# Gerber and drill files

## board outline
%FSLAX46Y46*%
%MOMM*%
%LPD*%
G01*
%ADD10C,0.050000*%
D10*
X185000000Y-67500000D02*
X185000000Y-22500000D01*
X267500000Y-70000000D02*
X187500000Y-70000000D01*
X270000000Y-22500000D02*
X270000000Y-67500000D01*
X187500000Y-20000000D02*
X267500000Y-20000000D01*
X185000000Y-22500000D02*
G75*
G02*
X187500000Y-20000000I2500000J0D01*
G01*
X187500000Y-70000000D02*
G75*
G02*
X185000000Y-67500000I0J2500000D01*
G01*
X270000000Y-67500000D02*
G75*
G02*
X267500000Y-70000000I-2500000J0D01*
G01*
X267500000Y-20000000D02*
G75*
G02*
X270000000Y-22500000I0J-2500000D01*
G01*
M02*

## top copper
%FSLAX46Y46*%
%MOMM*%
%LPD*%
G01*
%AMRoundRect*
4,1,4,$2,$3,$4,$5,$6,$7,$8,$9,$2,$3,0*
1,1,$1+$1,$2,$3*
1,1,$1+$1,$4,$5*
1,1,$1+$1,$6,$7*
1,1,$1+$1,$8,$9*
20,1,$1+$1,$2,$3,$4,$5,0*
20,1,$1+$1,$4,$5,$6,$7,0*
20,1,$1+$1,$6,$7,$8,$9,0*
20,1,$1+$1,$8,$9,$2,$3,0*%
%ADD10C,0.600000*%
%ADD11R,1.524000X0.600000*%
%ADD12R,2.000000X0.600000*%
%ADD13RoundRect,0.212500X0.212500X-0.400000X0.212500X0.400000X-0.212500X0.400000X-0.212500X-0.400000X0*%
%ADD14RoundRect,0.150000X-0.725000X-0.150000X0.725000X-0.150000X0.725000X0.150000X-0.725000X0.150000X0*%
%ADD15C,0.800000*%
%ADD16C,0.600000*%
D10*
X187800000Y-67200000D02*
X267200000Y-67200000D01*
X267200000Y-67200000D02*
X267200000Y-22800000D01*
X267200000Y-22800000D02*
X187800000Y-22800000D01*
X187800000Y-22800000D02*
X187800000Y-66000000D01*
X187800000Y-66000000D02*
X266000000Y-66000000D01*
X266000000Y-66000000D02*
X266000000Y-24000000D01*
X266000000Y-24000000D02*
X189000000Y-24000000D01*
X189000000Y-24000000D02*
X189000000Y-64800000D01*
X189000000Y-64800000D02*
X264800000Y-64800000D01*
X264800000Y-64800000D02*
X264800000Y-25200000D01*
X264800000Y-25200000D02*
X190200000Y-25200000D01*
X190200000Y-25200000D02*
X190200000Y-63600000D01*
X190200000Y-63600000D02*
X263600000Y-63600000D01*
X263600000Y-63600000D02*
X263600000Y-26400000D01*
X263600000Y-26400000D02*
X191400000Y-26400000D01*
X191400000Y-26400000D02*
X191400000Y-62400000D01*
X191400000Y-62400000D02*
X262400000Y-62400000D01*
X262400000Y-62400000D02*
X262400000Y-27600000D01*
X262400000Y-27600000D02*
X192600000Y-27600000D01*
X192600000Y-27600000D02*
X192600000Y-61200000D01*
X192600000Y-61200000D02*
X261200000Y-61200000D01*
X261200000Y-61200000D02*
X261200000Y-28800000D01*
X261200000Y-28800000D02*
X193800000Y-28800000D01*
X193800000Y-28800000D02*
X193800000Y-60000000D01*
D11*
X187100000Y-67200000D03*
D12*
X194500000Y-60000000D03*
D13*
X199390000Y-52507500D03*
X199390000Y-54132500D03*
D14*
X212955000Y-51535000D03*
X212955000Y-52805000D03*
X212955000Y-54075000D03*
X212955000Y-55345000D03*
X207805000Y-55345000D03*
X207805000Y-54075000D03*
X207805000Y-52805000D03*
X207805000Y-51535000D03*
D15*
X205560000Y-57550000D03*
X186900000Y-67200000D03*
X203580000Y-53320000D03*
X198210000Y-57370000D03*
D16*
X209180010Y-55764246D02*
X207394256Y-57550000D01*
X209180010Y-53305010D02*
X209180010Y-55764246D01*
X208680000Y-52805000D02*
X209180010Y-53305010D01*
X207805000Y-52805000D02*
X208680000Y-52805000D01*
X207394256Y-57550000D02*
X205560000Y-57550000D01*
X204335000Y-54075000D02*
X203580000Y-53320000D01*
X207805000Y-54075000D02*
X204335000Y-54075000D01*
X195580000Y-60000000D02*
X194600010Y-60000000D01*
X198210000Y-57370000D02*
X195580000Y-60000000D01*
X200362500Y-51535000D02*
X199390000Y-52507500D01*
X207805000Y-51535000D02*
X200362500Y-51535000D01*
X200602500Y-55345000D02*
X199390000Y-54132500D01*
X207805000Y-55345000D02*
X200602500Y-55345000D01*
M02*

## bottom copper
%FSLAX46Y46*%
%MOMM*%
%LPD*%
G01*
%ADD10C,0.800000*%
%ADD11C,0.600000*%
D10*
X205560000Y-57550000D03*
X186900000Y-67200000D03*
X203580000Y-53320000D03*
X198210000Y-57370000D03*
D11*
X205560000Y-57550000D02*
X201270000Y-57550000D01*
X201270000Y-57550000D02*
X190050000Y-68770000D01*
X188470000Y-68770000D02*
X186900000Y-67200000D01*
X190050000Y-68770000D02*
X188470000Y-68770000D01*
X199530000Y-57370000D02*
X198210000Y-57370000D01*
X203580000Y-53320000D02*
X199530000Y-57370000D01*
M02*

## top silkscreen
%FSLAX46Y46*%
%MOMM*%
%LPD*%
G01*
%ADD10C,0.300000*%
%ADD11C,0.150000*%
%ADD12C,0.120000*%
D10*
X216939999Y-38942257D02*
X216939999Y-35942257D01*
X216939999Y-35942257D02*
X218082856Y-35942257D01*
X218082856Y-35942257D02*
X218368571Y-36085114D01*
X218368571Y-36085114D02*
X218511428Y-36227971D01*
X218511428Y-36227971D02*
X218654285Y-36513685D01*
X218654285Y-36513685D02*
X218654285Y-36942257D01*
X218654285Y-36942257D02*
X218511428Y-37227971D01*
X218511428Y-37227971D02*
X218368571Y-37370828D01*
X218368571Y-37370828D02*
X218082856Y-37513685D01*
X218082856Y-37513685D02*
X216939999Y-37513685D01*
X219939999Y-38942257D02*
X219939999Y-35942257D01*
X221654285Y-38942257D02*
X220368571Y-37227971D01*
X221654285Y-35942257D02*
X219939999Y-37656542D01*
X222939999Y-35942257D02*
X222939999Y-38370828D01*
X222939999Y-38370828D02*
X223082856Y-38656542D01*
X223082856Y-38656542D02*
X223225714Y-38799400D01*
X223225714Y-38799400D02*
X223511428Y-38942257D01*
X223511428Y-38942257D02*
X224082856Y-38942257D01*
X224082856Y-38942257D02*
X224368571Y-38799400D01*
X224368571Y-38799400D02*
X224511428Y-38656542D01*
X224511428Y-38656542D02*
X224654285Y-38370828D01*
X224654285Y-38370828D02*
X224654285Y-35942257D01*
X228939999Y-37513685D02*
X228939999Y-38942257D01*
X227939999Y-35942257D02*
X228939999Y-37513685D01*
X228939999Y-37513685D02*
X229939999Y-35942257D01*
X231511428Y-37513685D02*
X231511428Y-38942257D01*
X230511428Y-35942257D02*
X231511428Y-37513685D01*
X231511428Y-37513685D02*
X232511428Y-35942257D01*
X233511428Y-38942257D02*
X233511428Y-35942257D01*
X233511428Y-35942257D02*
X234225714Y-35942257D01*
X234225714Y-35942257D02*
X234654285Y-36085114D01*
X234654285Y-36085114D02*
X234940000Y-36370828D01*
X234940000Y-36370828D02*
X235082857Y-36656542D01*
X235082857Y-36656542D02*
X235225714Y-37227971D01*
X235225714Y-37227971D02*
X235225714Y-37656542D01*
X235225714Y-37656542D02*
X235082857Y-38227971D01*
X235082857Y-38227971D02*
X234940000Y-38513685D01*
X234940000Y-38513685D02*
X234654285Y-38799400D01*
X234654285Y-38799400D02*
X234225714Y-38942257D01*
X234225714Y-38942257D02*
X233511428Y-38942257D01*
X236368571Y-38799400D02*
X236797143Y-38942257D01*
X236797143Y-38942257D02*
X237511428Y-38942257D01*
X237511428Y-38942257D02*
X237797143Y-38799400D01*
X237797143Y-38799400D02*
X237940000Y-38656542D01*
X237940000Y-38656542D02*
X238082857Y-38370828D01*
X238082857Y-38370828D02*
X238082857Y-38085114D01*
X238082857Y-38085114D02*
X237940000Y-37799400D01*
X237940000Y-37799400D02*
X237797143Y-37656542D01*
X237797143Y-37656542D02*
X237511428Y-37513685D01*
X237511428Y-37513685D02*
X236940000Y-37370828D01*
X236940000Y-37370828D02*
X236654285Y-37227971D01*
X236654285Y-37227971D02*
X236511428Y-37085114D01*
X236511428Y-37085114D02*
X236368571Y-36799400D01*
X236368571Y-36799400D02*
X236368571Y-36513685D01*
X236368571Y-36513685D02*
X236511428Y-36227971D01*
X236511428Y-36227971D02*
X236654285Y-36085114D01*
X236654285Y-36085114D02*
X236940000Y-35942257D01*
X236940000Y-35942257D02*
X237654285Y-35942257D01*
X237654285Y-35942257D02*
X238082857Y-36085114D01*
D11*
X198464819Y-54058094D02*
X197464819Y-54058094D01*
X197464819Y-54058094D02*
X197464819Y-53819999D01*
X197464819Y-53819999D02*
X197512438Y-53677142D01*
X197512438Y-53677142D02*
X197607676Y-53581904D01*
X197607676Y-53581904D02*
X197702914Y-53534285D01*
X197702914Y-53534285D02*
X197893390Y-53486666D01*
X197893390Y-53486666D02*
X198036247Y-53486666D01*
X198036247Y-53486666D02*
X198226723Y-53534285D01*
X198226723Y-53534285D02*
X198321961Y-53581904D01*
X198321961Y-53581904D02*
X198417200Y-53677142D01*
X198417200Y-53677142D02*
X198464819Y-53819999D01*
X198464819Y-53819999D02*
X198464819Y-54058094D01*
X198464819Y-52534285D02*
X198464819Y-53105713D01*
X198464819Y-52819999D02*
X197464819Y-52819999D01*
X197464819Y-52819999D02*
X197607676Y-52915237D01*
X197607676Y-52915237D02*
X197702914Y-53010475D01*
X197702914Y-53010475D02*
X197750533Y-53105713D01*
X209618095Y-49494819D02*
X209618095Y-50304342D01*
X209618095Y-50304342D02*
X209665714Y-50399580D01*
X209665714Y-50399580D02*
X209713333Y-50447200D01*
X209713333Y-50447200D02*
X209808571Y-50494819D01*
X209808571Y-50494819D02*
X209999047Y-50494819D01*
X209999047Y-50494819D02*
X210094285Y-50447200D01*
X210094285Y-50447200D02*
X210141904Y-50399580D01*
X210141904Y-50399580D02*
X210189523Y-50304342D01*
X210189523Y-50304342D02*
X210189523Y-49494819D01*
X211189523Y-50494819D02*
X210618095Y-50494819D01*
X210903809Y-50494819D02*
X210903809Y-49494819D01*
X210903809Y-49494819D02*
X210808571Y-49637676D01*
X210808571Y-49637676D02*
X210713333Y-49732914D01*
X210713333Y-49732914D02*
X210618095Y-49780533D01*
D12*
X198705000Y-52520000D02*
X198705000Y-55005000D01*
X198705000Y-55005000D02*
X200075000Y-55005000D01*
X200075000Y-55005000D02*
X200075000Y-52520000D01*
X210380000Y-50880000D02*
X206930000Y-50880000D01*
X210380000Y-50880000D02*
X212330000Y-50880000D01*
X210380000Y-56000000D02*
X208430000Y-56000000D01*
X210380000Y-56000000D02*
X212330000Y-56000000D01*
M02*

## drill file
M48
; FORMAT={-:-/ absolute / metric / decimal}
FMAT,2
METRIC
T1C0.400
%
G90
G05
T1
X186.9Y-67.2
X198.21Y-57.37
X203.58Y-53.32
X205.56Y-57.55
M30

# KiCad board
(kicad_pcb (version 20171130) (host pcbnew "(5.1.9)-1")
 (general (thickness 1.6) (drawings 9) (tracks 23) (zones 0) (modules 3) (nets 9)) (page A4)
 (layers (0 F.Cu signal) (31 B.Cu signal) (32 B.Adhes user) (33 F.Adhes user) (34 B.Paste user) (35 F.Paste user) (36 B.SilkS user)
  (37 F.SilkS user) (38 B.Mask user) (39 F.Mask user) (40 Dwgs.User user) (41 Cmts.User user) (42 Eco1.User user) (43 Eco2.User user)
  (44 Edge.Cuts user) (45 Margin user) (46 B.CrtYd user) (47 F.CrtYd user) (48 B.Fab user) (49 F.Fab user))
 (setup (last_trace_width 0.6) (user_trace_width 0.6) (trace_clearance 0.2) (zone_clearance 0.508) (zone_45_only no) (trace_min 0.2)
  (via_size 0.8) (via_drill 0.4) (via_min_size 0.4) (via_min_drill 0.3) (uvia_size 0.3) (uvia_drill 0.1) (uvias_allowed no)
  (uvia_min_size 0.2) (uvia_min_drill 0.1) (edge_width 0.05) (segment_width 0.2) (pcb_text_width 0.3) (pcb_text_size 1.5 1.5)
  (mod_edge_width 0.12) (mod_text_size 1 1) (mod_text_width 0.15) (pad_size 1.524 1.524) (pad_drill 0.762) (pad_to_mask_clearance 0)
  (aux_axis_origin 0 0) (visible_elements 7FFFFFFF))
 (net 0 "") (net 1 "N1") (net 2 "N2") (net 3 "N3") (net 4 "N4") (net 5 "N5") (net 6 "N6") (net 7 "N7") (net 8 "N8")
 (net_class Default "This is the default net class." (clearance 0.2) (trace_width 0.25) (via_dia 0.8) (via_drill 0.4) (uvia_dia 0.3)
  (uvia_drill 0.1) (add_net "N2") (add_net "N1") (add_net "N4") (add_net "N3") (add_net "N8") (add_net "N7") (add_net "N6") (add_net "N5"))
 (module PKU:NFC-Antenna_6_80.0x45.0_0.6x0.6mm (layer F.Cu) (at 227.5 45)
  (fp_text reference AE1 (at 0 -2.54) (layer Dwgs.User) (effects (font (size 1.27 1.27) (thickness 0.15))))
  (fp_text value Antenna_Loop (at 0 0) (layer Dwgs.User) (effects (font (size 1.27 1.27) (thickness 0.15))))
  (fp_line (start -39.7 22.2) (end 39.7 22.2) (layer F.Cu) (width 0.6))
  (fp_line (start 39.7 22.2) (end 39.7 -22.2) (layer F.Cu) (width 0.6))
  (fp_line (start 39.7 -22.2) (end -39.7 -22.2) (layer F.Cu) (width 0.6))
  (fp_line (start -39.7 -22.2) (end -39.7 21) (layer F.Cu) (width 0.6))
  (fp_line (start -39.7 21) (end 38.5 21) (layer F.Cu) (width 0.6))
  (fp_line (start 38.5 21) (end 38.5 -21) (layer F.Cu) (width 0.6))
  (fp_line (start 38.5 -21) (end -38.5 -21) (layer F.Cu) (width 0.6))
  (fp_line (start -38.5 -21) (end -38.5 19.8) (layer F.Cu) (width 0.6))
  (fp_line (start -38.5 19.8) (end 37.3 19.8) (layer F.Cu) (width 0.6))
  (fp_line (start 37.3 19.8) (end 37.3 -19.8) (layer F.Cu) (width 0.6))
  (fp_line (start 37.3 -19.8) (end -37.3 -19.8) (layer F.Cu) (width 0.6))
  (fp_line (start -37.3 -19.8) (end -37.3 18.6) (layer F.Cu) (width 0.6))
  (fp_line (start -37.3 18.6) (end 36.1 18.6) (layer F.Cu) (width 0.6))
  (fp_line (start 36.1 18.6) (end 36.1 -18.6) (layer F.Cu) (width 0.6))
  (fp_line (start 36.1 -18.6) (end -36.1 -18.6) (layer F.Cu) (width 0.6))
  (fp_line (start -36.1 -18.6) (end -36.1 17.4) (layer F.Cu) (width 0.6))
  (fp_line (start -36.1 17.4) (end 34.9 17.4) (layer F.Cu) (width 0.6))
  (fp_line (start 34.9 17.4) (end 34.9 -17.4) (layer F.Cu) (width 0.6))
  (fp_line (start 34.9 -17.4) (end -34.9 -17.4) (layer F.Cu) (width 0.6))
  (fp_line (start -34.9 -17.4) (end -34.9 16.2) (layer F.Cu) (width 0.6))
  (fp_line (start -34.9 16.2) (end 33.7 16.2) (layer F.Cu) (width 0.6))
  (fp_line (start 33.7 16.2) (end 33.7 -16.2) (layer F.Cu) (width 0.6))
  (fp_line (start 33.7 -16.2) (end -33.7 -16.2) (layer F.Cu) (width 0.6))
  (fp_line (start -33.7 -16.2) (end -33.7 15) (layer F.Cu) (width 0.6))
  (pad 2 smd rect (at -40.4 22.2 90) (size 0.6 1.524) (layers F.Cu) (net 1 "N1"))
  (pad 1 smd rect (at -33 15 90) (size 0.6 2) (layers F.Cu) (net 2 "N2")))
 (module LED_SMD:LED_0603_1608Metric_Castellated (layer F.Cu) (at 199.39 53.32 90)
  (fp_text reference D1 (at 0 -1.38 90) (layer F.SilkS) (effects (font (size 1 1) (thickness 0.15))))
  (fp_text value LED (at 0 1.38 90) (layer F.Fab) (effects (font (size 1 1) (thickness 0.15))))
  (fp_line (start 0.8 -0.685) (end -1.685 -0.685) (layer F.SilkS) (width 0.12))
  (fp_line (start -1.685 -0.685) (end -1.685 0.685) (layer F.SilkS) (width 0.12))
  (fp_line (start -1.685 0.685) (end 0.8 0.685) (layer F.SilkS) (width 0.12))
  (pad 2 smd roundrect (at 0.8125 0 90) (size 1.225 0.85) (layers F.Cu F.Paste F.Mask) (roundrect_rratio 0.25) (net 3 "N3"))
  (pad 1 smd roundrect (at -0.8125 0 90) (size 1.225 0.85) (layers F.Cu F.Paste F.Mask) (roundrect_rratio 0.25) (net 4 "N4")))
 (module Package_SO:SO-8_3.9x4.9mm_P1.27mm (layer F.Cu) (at 210.38 53.44)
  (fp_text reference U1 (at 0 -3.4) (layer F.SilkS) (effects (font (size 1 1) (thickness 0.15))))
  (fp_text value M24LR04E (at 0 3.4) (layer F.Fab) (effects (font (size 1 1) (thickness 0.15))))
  (fp_line (start 0 -2.56) (end -3.45 -2.56) (layer F.SilkS) (width 0.12))
  (fp_line (start 0 -2.56) (end 1.95 -2.56) (layer F.SilkS) (width 0.12))
  (fp_line (start 0 2.56) (end -1.95 2.56) (layer F.SilkS) (width 0.12))
  (fp_line (start 0 2.56) (end 1.95 2.56) (layer F.SilkS) (width 0.12))
  (pad 8 smd roundrect (at 2.575 -1.905) (size 1.75 0.6) (layers F.Cu F.Paste F.Mask) (roundrect_rratio 0.25) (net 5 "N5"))
  (pad 7 smd roundrect (at 2.575 -0.635) (size 1.75 0.6) (layers F.Cu F.Paste F.Mask) (roundrect_rratio 0.25) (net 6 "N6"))
  (pad 6 smd roundrect (at 2.575 0.635) (size 1.75 0.6) (layers F.Cu F.Paste F.Mask) (roundrect_rratio 0.25) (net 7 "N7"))
  (pad 5 smd roundrect (at 2.575 1.905) (size 1.75 0.6) (layers F.Cu F.Paste F.Mask) (roundrect_rratio 0.25) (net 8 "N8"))
  (pad 4 smd roundrect (at -2.575 1.905) (size 1.75 0.6) (layers F.Cu F.Paste F.Mask) (roundrect_rratio 0.25) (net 4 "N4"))
  (pad 3 smd roundrect (at -2.575 0.635) (size 1.75 0.6) (layers F.Cu F.Paste F.Mask) (roundrect_rratio 0.25) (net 2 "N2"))
  (pad 2 smd roundrect (at -2.575 -0.635) (size 1.75 0.6) (layers F.Cu F.Paste F.Mask) (roundrect_rratio 0.25) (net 1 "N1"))
  (pad 1 smd roundrect (at -2.575 -1.905) (size 1.75 0.6) (layers F.Cu F.Paste F.Mask) (roundrect_rratio 0.25) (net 3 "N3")))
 (gr_line (start 185 67.5) (end 185 22.5) (layer Edge.Cuts) (width 0.05))
 (gr_line (start 267.5 70) (end 187.5 70) (layer Edge.Cuts) (width 0.05))
 (gr_line (start 270 22.5) (end 270 67.5) (layer Edge.Cuts) (width 0.05))
 (gr_line (start 187.5 20) (end 267.5 20) (layer Edge.Cuts) (width 0.05))
 (gr_arc (start 187.5 22.5) (end 187.5 20) (angle -90) (layer Edge.Cuts) (width 0.05))
 (gr_arc (start 187.5 67.5) (end 185 67.5) (angle -90) (layer Edge.Cuts) (width 0.05))
 (gr_arc (start 267.5 67.5) (end 267.5 70) (angle -90) (layer Edge.Cuts) (width 0.05))
 (gr_arc (start 267.5 22.5) (end 270 22.5) (angle -90) (layer Edge.Cuts) (width 0.05))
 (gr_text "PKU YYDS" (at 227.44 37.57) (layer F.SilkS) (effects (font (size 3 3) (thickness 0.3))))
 (segment (start 209.18001 55.764246) (end 207.394256 57.55) (width 0.6) (layer F.Cu) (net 1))
 (segment (start 209.18001 53.30501) (end 209.18001 55.764246) (width 0.6) (layer F.Cu) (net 1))
 (segment (start 208.68 52.805) (end 209.18001 53.30501) (width 0.6) (layer F.Cu) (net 1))
 (segment (start 207.805 52.805) (end 208.68 52.805) (width 0.6) (layer F.Cu) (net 1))
 (via (at 205.56 57.55) (size 0.8) (drill 0.4) (layers F.Cu B.Cu) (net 1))
 (segment (start 207.394256 57.55) (end 205.56 57.55) (width 0.6) (layer F.Cu) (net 1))
 (segment (start 205.56 57.55) (end 201.27 57.55) (width 0.6) (layer B.Cu) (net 1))
 (segment (start 201.27 57.55) (end 190.05 68.77) (width 0.6) (layer B.Cu) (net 1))
 (via (at 186.9 67.2) (size 0.8) (drill 0.4) (layers F.Cu B.Cu) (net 1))
 (segment (start 188.47 68.77) (end 186.9 67.2) (width 0.6) (layer B.Cu) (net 1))
 (segment (start 190.05 68.77) (end 188.47 68.77) (width 0.6) (layer B.Cu) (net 1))
 (via (at 203.58 53.32) (size 0.8) (drill 0.4) (layers F.Cu B.Cu) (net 2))
 (segment (start 204.335 54.075) (end 203.58 53.32) (width 0.6) (layer F.Cu) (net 2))
 (segment (start 207.805 54.075) (end 204.335 54.075) (width 0.6) (layer F.Cu) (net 2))
 (via (at 198.21 57.37) (size 0.8) (drill 0.4) (layers F.Cu B.Cu) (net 2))
 (segment (start 199.53 57.37) (end 198.21 57.37) (width 0.6) (layer B.Cu) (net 2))
 (segment (start 203.58 53.32) (end 199.53 57.37) (width 0.6) (layer B.Cu) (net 2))
 (segment (start 195.58 60) (end 194.60001 60) (width 0.6) (layer F.Cu) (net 2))
 (segment (start 198.21 57.37) (end 195.58 60) (width 0.6) (layer F.Cu) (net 2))
 (segment (start 200.3625 51.535) (end 199.39 52.5075) (width 0.6) (layer F.Cu) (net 3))
 (segment (start 207.805 51.535) (end 200.3625 51.535) (width 0.6) (layer F.Cu) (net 3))
 (segment (start 200.6025 55.345) (end 199.39 54.1325) (width 0.6) (layer F.Cu) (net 4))
 (segment (start 207.805 55.345) (end 200.6025 55.345) (width 0.6) (layer F.Cu) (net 4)))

